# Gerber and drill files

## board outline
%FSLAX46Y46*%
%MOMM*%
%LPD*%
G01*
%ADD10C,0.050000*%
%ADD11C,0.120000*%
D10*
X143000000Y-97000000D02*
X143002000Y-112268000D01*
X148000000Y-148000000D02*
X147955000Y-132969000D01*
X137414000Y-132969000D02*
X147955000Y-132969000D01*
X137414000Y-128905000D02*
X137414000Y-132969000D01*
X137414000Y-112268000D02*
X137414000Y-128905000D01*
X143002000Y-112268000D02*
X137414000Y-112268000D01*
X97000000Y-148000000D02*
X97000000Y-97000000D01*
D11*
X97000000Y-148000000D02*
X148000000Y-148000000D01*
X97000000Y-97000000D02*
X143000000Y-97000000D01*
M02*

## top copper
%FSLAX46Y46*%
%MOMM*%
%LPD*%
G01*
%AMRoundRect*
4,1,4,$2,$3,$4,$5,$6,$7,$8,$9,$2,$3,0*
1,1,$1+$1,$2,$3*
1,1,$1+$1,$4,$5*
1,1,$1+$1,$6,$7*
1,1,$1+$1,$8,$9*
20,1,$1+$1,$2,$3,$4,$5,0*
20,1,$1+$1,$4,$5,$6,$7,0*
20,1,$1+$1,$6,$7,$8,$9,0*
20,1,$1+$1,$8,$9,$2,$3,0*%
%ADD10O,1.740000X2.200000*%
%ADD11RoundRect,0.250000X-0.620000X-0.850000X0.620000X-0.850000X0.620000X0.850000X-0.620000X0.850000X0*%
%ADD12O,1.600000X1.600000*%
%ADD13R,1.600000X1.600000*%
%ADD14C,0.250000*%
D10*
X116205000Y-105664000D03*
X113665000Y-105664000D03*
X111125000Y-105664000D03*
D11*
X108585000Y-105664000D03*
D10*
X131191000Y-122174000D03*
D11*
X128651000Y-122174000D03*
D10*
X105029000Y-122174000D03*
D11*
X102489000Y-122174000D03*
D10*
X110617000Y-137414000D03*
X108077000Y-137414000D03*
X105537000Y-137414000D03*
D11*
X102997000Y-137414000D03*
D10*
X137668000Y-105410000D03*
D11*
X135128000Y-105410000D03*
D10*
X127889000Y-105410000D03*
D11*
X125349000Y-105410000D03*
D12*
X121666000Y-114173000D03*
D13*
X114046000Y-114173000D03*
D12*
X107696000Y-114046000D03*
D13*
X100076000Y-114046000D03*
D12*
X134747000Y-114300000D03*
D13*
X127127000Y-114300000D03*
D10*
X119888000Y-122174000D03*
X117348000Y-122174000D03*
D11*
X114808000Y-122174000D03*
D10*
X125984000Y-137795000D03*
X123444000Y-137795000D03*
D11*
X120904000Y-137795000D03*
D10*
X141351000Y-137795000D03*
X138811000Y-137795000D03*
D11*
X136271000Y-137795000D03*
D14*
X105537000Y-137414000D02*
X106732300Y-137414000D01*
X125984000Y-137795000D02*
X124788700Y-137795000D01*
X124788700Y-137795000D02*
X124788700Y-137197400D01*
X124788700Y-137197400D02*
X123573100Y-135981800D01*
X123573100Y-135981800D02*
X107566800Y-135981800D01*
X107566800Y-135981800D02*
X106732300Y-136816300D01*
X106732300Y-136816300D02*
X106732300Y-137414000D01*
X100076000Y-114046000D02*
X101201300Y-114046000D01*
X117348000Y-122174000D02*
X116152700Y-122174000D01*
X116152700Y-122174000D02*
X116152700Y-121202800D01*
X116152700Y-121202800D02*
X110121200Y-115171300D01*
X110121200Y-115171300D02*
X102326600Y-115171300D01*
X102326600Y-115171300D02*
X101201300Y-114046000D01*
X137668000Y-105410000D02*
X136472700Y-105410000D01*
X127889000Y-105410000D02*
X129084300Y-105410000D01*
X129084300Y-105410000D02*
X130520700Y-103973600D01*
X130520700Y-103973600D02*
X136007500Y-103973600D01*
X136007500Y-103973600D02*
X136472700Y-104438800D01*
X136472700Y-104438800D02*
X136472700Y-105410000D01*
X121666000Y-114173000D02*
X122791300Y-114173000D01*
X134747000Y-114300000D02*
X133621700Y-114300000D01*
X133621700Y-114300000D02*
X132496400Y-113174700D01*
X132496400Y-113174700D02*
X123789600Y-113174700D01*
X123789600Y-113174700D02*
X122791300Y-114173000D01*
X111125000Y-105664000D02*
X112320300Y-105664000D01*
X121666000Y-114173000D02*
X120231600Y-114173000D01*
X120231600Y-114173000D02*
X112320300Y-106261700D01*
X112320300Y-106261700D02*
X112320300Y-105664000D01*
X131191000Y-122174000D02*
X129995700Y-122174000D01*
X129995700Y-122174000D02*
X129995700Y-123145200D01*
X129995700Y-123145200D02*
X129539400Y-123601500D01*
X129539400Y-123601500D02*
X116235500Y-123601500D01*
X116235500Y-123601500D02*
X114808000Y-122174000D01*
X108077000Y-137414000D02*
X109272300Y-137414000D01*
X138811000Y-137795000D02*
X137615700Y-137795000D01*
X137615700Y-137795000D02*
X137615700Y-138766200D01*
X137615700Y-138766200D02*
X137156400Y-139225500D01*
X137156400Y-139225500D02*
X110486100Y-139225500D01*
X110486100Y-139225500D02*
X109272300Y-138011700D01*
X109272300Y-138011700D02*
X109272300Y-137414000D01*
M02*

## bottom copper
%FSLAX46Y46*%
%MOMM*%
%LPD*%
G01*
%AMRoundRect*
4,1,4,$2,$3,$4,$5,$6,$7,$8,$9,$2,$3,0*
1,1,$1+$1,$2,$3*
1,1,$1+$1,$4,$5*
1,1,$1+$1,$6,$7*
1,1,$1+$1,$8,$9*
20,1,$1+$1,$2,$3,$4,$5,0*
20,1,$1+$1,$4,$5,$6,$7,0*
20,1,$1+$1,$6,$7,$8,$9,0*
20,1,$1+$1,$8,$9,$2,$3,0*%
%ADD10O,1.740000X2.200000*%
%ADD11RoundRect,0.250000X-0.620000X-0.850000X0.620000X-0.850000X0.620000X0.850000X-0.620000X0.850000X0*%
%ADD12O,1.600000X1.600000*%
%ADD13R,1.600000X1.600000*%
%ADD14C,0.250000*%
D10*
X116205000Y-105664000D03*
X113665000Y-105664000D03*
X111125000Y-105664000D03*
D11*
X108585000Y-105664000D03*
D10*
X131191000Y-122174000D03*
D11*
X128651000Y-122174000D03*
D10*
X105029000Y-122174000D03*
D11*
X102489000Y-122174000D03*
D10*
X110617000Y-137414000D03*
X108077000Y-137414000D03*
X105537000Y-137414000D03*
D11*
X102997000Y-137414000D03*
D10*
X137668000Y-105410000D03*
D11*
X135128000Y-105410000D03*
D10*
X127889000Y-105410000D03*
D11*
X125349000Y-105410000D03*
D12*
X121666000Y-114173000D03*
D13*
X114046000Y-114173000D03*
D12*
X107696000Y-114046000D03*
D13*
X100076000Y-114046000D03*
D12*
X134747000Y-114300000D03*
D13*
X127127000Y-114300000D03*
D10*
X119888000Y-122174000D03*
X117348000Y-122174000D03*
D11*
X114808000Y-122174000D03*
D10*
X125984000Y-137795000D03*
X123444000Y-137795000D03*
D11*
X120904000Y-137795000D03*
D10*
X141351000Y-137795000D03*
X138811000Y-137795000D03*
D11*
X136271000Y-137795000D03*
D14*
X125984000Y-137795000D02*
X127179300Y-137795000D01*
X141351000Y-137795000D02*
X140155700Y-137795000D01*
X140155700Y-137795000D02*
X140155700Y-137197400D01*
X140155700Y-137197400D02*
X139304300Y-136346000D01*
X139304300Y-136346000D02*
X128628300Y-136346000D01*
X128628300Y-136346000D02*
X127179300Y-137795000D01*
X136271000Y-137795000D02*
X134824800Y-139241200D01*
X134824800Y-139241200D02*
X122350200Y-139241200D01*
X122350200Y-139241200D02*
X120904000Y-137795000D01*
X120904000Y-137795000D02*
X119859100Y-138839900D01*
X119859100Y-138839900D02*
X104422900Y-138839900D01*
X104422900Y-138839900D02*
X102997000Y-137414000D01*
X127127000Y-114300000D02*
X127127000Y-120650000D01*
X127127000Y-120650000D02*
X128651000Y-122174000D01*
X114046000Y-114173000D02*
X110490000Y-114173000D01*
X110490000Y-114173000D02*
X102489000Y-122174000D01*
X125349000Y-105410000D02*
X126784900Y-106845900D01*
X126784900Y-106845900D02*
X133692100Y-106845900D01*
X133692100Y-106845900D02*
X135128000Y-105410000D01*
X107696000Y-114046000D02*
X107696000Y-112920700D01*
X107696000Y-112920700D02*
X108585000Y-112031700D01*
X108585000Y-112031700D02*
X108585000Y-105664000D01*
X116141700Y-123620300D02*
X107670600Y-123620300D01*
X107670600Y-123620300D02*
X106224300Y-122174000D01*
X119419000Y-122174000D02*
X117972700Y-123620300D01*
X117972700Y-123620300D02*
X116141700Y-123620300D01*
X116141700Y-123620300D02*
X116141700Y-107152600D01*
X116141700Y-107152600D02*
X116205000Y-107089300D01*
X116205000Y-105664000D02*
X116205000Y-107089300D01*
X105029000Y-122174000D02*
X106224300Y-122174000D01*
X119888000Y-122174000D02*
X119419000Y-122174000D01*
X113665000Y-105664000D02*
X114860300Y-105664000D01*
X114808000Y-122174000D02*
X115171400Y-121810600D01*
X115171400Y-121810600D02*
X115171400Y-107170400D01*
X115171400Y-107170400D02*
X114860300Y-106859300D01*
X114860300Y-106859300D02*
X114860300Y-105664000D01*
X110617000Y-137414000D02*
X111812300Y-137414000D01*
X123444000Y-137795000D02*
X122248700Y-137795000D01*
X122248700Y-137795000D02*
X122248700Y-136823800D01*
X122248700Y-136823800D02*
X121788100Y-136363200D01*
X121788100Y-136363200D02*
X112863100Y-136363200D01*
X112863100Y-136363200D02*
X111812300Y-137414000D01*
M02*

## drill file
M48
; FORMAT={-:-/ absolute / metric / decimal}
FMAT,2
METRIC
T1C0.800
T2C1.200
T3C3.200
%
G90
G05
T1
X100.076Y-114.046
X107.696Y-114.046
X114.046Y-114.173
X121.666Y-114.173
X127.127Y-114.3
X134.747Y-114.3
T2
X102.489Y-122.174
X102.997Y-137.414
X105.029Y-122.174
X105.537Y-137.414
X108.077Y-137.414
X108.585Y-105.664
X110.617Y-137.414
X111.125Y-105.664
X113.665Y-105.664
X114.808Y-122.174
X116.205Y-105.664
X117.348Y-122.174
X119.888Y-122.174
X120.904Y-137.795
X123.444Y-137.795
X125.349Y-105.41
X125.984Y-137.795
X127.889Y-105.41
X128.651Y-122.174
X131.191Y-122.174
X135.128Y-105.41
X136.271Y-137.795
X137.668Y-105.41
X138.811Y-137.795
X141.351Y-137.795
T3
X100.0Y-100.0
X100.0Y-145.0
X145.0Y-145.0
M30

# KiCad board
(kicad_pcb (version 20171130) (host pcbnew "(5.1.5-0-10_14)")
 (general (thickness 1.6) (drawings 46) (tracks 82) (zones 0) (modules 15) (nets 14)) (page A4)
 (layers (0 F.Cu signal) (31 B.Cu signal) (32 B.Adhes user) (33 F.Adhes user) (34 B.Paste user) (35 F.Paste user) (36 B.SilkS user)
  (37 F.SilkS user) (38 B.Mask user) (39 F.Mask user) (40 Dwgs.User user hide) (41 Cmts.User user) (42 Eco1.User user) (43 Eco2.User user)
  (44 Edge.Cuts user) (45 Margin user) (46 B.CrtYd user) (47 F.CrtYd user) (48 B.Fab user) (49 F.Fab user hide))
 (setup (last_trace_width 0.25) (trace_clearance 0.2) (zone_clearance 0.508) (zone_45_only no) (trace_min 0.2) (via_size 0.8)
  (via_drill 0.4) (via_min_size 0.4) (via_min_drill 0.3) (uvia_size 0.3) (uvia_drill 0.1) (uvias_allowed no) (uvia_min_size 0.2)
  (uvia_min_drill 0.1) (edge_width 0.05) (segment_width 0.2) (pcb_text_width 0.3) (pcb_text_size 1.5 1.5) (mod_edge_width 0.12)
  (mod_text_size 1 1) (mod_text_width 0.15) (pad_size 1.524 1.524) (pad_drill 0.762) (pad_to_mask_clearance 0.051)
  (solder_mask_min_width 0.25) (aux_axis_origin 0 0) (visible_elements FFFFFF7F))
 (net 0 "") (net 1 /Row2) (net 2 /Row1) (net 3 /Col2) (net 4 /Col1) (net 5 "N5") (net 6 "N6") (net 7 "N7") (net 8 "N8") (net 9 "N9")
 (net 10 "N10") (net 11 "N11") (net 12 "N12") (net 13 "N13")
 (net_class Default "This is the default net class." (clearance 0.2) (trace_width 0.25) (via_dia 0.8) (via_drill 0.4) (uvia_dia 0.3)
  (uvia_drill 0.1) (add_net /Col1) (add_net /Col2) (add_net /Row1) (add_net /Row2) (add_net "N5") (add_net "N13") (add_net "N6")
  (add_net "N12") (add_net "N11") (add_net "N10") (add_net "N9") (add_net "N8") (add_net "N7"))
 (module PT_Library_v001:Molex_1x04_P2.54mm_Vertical (layer F.Cu) (at 108.585 105.664)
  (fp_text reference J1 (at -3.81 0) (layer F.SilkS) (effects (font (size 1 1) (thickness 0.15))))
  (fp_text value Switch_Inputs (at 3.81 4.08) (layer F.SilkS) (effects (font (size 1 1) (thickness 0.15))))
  (pad 4 thru_hole oval (at 7.62 0) (size 1.74 2.2) (drill 1.2) (layers *.Cu *.Mask) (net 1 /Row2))
  (pad 3 thru_hole oval (at 5.08 0) (size 1.74 2.2) (drill 1.2) (layers *.Cu *.Mask) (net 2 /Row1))
  (pad 2 thru_hole oval (at 2.54 0) (size 1.74 2.2) (drill 1.2) (layers *.Cu *.Mask) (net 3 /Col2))
  (pad 1 thru_hole roundrect (at 0 0) (size 1.74 2.2) (drill 1.2) (layers *.Cu *.Mask) (roundrect_rratio 0.143678) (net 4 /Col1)))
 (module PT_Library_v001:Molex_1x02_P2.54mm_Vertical (layer F.Cu) (at 128.651 122.174)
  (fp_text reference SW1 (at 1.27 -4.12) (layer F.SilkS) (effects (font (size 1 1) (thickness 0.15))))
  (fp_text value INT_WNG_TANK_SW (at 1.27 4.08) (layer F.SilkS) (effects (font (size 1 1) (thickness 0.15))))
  (pad 2 thru_hole oval (at 2.54 0) (size 1.74 2.2) (drill 1.2) (layers *.Cu *.Mask) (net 2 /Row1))
  (pad 1 thru_hole roundrect (at 0 0) (size 1.74 2.2) (drill 1.2) (layers *.Cu *.Mask) (roundrect_rratio 0.143678) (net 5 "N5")))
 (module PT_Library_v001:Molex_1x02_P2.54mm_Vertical (layer F.Cu) (at 102.489 122.174)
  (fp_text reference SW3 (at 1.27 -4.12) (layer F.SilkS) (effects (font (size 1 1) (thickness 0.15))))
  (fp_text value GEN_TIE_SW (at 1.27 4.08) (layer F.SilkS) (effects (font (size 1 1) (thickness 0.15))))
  (pad 2 thru_hole oval (at 2.54 0) (size 1.74 2.2) (drill 1.2) (layers *.Cu *.Mask) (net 1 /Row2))
  (pad 1 thru_hole roundrect (at 0 0) (size 1.74 2.2) (drill 1.2) (layers *.Cu *.Mask) (roundrect_rratio 0.143678) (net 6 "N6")))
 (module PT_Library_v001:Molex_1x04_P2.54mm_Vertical (layer F.Cu) (at 102.997 137.414)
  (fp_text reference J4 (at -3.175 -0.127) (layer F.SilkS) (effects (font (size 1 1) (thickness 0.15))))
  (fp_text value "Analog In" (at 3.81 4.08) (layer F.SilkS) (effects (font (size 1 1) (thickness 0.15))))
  (pad 4 thru_hole oval (at 7.62 0) (size 1.74 2.2) (drill 1.2) (layers *.Cu *.Mask) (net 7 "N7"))
  (pad 3 thru_hole oval (at 5.08 0) (size 1.74 2.2) (drill 1.2) (layers *.Cu *.Mask) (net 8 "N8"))
  (pad 2 thru_hole oval (at 2.54 0) (size 1.74 2.2) (drill 1.2) (layers *.Cu *.Mask) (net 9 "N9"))
  (pad 1 thru_hole roundrect (at 0 0) (size 1.74 2.2) (drill 1.2) (layers *.Cu *.Mask) (roundrect_rratio 0.143678) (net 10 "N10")))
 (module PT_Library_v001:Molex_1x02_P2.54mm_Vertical (layer F.Cu) (at 135.128 105.41)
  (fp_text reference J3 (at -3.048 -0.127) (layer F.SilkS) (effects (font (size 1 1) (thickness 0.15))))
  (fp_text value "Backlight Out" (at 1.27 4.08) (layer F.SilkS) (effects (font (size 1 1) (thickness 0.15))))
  (pad 2 thru_hole oval (at 2.54 0) (size 1.74 2.2) (drill 1.2) (layers *.Cu *.Mask) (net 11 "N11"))
  (pad 1 thru_hole roundrect (at 0 0) (size 1.74 2.2) (drill 1.2) (layers *.Cu *.Mask) (roundrect_rratio 0.143678) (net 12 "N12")))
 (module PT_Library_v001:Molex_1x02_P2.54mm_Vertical (layer F.Cu) (at 125.349 105.41)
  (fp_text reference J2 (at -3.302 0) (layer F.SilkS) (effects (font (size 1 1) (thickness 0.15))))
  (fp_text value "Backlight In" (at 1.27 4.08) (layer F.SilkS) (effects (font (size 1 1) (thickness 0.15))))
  (pad 2 thru_hole oval (at 2.54 0) (size 1.74 2.2) (drill 1.2) (layers *.Cu *.Mask) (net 11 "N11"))
  (pad 1 thru_hole roundrect (at 0 0) (size 1.74 2.2) (drill 1.2) (layers *.Cu *.Mask) (roundrect_rratio 0.143678) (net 12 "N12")))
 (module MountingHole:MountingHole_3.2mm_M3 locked (layer F.Cu) (at 145 145)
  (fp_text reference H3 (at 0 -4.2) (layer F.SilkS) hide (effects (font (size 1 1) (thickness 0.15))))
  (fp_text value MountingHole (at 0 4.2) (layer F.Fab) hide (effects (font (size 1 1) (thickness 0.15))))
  (pad 1 np_thru_hole circle (at 0 0) (size 3.2 3.2) (drill 3.2) (layers *.Cu *.Mask)))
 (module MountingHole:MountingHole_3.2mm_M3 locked (layer F.Cu) (at 100 100)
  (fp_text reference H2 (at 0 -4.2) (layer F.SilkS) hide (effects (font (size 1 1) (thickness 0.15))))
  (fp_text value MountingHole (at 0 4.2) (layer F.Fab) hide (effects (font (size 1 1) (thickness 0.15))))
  (pad 1 np_thru_hole circle (at 0 0) (size 3.2 3.2) (drill 3.2) (layers *.Cu *.Mask)))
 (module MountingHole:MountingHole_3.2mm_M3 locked (layer F.Cu) (at 100 145)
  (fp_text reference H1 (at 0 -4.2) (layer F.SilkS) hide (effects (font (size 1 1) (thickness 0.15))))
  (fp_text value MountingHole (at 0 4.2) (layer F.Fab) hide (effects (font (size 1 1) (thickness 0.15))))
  (pad 1 np_thru_hole circle (at 0 0) (size 3.2 3.2) (drill 3.2) (layers *.Cu *.Mask)))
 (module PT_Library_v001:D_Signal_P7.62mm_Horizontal (layer F.Cu) (at 114.046 114.173)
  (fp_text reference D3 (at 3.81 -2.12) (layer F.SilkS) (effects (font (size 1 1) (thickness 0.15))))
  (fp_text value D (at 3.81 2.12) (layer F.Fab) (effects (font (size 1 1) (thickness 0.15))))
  (pad 2 thru_hole oval (at 7.62 0) (size 1.6 1.6) (drill 0.8) (layers *.Cu *.Mask) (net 3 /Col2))
  (pad 1 thru_hole rect (at 0 0) (size 1.6 1.6) (drill 0.8) (layers *.Cu *.Mask) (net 6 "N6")))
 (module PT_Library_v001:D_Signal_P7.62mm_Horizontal (layer F.Cu) (at 100.076 114.046)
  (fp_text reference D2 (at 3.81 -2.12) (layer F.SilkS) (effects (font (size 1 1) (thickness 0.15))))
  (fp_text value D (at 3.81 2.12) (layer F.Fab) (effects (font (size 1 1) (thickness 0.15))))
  (pad 2 thru_hole oval (at 7.62 0) (size 1.6 1.6) (drill 0.8) (layers *.Cu *.Mask) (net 4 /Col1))
  (pad 1 thru_hole rect (at 0 0) (size 1.6 1.6) (drill 0.8) (layers *.Cu *.Mask) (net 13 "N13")))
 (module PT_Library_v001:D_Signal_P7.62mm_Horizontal (layer F.Cu) (at 127.127 114.3)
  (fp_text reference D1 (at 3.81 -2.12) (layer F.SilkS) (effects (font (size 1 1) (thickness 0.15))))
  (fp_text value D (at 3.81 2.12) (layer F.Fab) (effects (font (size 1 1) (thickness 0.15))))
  (pad 2 thru_hole oval (at 7.62 0) (size 1.6 1.6) (drill 0.8) (layers *.Cu *.Mask) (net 3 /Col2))
  (pad 1 thru_hole rect (at 0 0) (size 1.6 1.6) (drill 0.8) (layers *.Cu *.Mask) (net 5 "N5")))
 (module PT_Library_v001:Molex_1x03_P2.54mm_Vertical (layer F.Cu) (at 114.808 122.174)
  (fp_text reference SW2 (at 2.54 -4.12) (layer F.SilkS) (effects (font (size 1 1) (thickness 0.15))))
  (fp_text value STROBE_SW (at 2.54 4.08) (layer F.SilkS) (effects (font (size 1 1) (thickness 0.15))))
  (pad 3 thru_hole oval (at 5.08 0) (size 1.74 2.2) (drill 1.2) (layers *.Cu *.Mask) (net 1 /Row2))
  (pad 2 thru_hole oval (at 2.54 0) (size 1.74 2.2) (drill 1.2) (layers *.Cu *.Mask) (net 13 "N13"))
  (pad 1 thru_hole roundrect (at 0 0) (size 1.74 2.2) (drill 1.2) (layers *.Cu *.Mask) (roundrect_rratio 0.143678) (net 2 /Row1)))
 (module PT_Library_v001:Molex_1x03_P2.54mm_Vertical (layer F.Cu) (at 120.904 137.795)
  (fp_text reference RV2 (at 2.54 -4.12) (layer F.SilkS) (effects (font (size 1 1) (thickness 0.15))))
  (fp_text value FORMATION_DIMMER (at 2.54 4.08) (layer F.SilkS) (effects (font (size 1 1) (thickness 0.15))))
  (pad 3 thru_hole oval (at 5.08 0) (size 1.74 2.2) (drill 1.2) (layers *.Cu *.Mask) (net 9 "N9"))
  (pad 2 thru_hole oval (at 2.54 0) (size 1.74 2.2) (drill 1.2) (layers *.Cu *.Mask) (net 7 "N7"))
  (pad 1 thru_hole roundrect (at 0 0) (size 1.74 2.2) (drill 1.2) (layers *.Cu *.Mask) (roundrect_rratio 0.143678) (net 10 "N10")))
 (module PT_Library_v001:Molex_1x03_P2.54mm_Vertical (layer F.Cu) (at 136.271 137.795)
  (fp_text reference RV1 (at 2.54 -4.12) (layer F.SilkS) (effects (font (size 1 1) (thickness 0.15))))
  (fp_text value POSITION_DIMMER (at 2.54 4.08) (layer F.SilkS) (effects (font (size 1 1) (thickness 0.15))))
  (pad 3 thru_hole oval (at 5.08 0) (size 1.74 2.2) (drill 1.2) (layers *.Cu *.Mask) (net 9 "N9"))
  (pad 2 thru_hole oval (at 2.54 0) (size 1.74 2.2) (drill 1.2) (layers *.Cu *.Mask) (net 8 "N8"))
  (pad 1 thru_hole roundrect (at 0 0) (size 1.74 2.2) (drill 1.2) (layers *.Cu *.Mask) (roundrect_rratio 0.143678) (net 10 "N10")))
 (gr_line (start 143 97) (end 143.002 112.268) (layer Edge.Cuts) (width 0.05))
 (gr_line (start 148 148) (end 147.955 132.969) (layer Edge.Cuts) (width 0.05))
 (gr_line (start 137.414 132.969) (end 147.955 132.969) (layer Edge.Cuts) (width 0.05))
 (gr_line (start 137.414 128.905) (end 137.414 132.969) (layer Edge.Cuts) (width 0.05))
 (gr_line (start 137.414 112.268) (end 137.414 128.905) (layer Edge.Cuts) (width 0.05))
 (gr_line (start 143.002 112.268) (end 137.414 112.268) (layer Edge.Cuts) (width 0.05))
 (gr_line (start 97 148) (end 97 97) (layer Edge.Cuts) (width 0.05))
 (gr_line (start 97 148) (end 148 148) (layer Edge.Cuts) (width 0.12))
 (gr_line (start 97 97) (end 143 97) (layer Edge.Cuts) (width 0.12))
 (segment (start 105.537 137.414) (end 106.7323 137.414) (width 0.25) (layer F.Cu) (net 9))
 (segment (start 125.984 137.795) (end 124.7887 137.795) (width 0.25) (layer F.Cu) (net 9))
 (segment (start 124.7887 137.795) (end 124.7887 137.1974) (width 0.25) (layer F.Cu) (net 9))
 (segment (start 124.7887 137.1974) (end 123.5731 135.9818) (width 0.25) (layer F.Cu) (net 9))
 (segment (start 123.5731 135.9818) (end 107.5668 135.9818) (width 0.25) (layer F.Cu) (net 9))
 (segment (start 107.5668 135.9818) (end 106.7323 136.8163) (width 0.25) (layer F.Cu) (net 9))
 (segment (start 106.7323 136.8163) (end 106.7323 137.414) (width 0.25) (layer F.Cu) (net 9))
 (segment (start 125.984 137.795) (end 127.1793 137.795) (width 0.25) (layer B.Cu) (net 9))
 (segment (start 141.351 137.795) (end 140.1557 137.795) (width 0.25) (layer B.Cu) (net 9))
 (segment (start 140.1557 137.795) (end 140.1557 137.1974) (width 0.25) (layer B.Cu) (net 9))
 (segment (start 140.1557 137.1974) (end 139.3043 136.346) (width 0.25) (layer B.Cu) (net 9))
 (segment (start 139.3043 136.346) (end 128.6283 136.346) (width 0.25) (layer B.Cu) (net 9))
 (segment (start 128.6283 136.346) (end 127.1793 137.795) (width 0.25) (layer B.Cu) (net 9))
 (segment (start 100.076 114.046) (end 101.2013 114.046) (width 0.25) (layer F.Cu) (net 13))
 (segment (start 117.348 122.174) (end 116.1527 122.174) (width 0.25) (layer F.Cu) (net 13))
 (segment (start 116.1527 122.174) (end 116.1527 121.2028) (width 0.25) (layer F.Cu) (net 13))
 (segment (start 116.1527 121.2028) (end 110.1212 115.1713) (width 0.25) (layer F.Cu) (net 13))
 (segment (start 110.1212 115.1713) (end 102.3266 115.1713) (width 0.25) (layer F.Cu) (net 13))
 (segment (start 102.3266 115.1713) (end 101.2013 114.046) (width 0.25) (layer F.Cu) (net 13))
 (segment (start 136.271 137.795) (end 134.8248 139.2412) (width 0.25) (layer B.Cu) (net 10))
 (segment (start 134.8248 139.2412) (end 122.3502 139.2412) (width 0.25) (layer B.Cu) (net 10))
 (segment (start 122.3502 139.2412) (end 120.904 137.795) (width 0.25) (layer B.Cu) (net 10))
 (segment (start 120.904 137.795) (end 119.8591 138.8399) (width 0.25) (layer B.Cu) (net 10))
 (segment (start 119.8591 138.8399) (end 104.4229 138.8399) (width 0.25) (layer B.Cu) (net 10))
 (segment (start 104.4229 138.8399) (end 102.997 137.414) (width 0.25) (layer B.Cu) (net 10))
 (segment (start 127.127 114.3) (end 127.127 120.65) (width 0.25) (layer B.Cu) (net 5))
 (segment (start 127.127 120.65) (end 128.651 122.174) (width 0.25) (layer B.Cu) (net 5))
 (segment (start 114.046 114.173) (end 110.49 114.173) (width 0.25) (layer B.Cu) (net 6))
 (segment (start 110.49 114.173) (end 102.489 122.174) (width 0.25) (layer B.Cu) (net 6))
 (segment (start 137.668 105.41) (end 136.4727 105.41) (width 0.25) (layer F.Cu) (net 11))
 (segment (start 127.889 105.41) (end 129.0843 105.41) (width 0.25) (layer F.Cu) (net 11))
 (segment (start 129.0843 105.41) (end 130.5207 103.9736) (width 0.25) (layer F.Cu) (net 11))
 (segment (start 130.5207 103.9736) (end 136.0075 103.9736) (width 0.25) (layer F.Cu) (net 11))
 (segment (start 136.0075 103.9736) (end 136.4727 104.4388) (width 0.25) (layer F.Cu) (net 11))
 (segment (start 136.4727 104.4388) (end 136.4727 105.41) (width 0.25) (layer F.Cu) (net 11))
 (segment (start 125.349 105.41) (end 126.7849 106.8459) (width 0.25) (layer B.Cu) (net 12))
 (segment (start 126.7849 106.8459) (end 133.6921 106.8459) (width 0.25) (layer B.Cu) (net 12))
 (segment (start 133.6921 106.8459) (end 135.128 105.41) (width 0.25) (layer B.Cu) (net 12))
 (segment (start 121.666 114.173) (end 122.7913 114.173) (width 0.25) (layer F.Cu) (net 3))
 (segment (start 134.747 114.3) (end 133.6217 114.3) (width 0.25) (layer F.Cu) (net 3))
 (segment (start 133.6217 114.3) (end 132.4964 113.1747) (width 0.25) (layer F.Cu) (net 3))
 (segment (start 132.4964 113.1747) (end 123.7896 113.1747) (width 0.25) (layer F.Cu) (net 3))
 (segment (start 123.7896 113.1747) (end 122.7913 114.173) (width 0.25) (layer F.Cu) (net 3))
 (segment (start 111.125 105.664) (end 112.3203 105.664) (width 0.25) (layer F.Cu) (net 3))
 (segment (start 121.666 114.173) (end 120.2316 114.173) (width 0.25) (layer F.Cu) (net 3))
 (segment (start 120.2316 114.173) (end 112.3203 106.2617) (width 0.25) (layer F.Cu) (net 3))
 (segment (start 112.3203 106.2617) (end 112.3203 105.664) (width 0.25) (layer F.Cu) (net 3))
 (segment (start 107.696 114.046) (end 107.696 112.9207) (width 0.25) (layer B.Cu) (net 4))
 (segment (start 107.696 112.9207) (end 108.585 112.0317) (width 0.25) (layer B.Cu) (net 4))
 (segment (start 108.585 112.0317) (end 108.585 105.664) (width 0.25) (layer B.Cu) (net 4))
 (segment (start 116.1417 123.6203) (end 107.6706 123.6203) (width 0.25) (layer B.Cu) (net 1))
 (segment (start 107.6706 123.6203) (end 106.2243 122.174) (width 0.25) (layer B.Cu) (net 1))
 (segment (start 119.419 122.174) (end 117.9727 123.6203) (width 0.25) (layer B.Cu) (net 1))
 (segment (start 117.9727 123.6203) (end 116.1417 123.6203) (width 0.25) (layer B.Cu) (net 1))
 (segment (start 116.1417 123.6203) (end 116.1417 107.1526) (width 0.25) (layer B.Cu) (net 1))
 (segment (start 116.1417 107.1526) (end 116.205 107.0893) (width 0.25) (layer B.Cu) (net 1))
 (segment (start 116.205 105.664) (end 116.205 107.0893) (width 0.25) (layer B.Cu) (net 1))
 (segment (start 105.029 122.174) (end 106.2243 122.174) (width 0.25) (layer B.Cu) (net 1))
 (segment (start 119.888 122.174) (end 119.419 122.174) (width 0.25) (layer B.Cu) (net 1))
 (segment (start 131.191 122.174) (end 129.9957 122.174) (width 0.25) (layer F.Cu) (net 2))
 (segment (start 129.9957 122.174) (end 129.9957 123.1452) (width 0.25) (layer F.Cu) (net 2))
 (segment (start 129.9957 123.1452) (end 129.5394 123.6015) (width 0.25) (layer F.Cu) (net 2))
 (segment (start 129.5394 123.6015) (end 116.2355 123.6015) (width 0.25) (layer F.Cu) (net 2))
 (segment (start 116.2355 123.6015) (end 114.808 122.174) (width 0.25) (layer F.Cu) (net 2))
 (segment (start 113.665 105.664) (end 114.8603 105.664) (width 0.25) (layer B.Cu) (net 2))
 (segment (start 114.808 122.174) (end 115.1714 121.8106) (width 0.25) (layer B.Cu) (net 2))
 (segment (start 115.1714 121.8106) (end 115.1714 107.1704) (width 0.25) (layer B.Cu) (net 2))
 (segment (start 115.1714 107.1704) (end 114.8603 106.8593) (width 0.25) (layer B.Cu) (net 2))
 (segment (start 114.8603 106.8593) (end 114.8603 105.664) (width 0.25) (layer B.Cu) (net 2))
 (segment (start 110.617 137.414) (end 111.8123 137.414) (width 0.25) (layer B.Cu) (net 7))
 (segment (start 123.444 137.795) (end 122.2487 137.795) (width 0.25) (layer B.Cu) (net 7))
 (segment (start 122.2487 137.795) (end 122.2487 136.8238) (width 0.25) (layer B.Cu) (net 7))
 (segment (start 122.2487 136.8238) (end 121.7881 136.3632) (width 0.25) (layer B.Cu) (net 7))
 (segment (start 121.7881 136.3632) (end 112.8631 136.3632) (width 0.25) (layer B.Cu) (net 7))
 (segment (start 112.8631 136.3632) (end 111.8123 137.414) (width 0.25) (layer B.Cu) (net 7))
 (segment (start 108.077 137.414) (end 109.2723 137.414) (width 0.25) (layer F.Cu) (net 8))
 (segment (start 138.811 137.795) (end 137.6157 137.795) (width 0.25) (layer F.Cu) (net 8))
 (segment (start 137.6157 137.795) (end 137.6157 138.7662) (width 0.25) (layer F.Cu) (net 8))
 (segment (start 137.6157 138.7662) (end 137.1564 139.2255) (width 0.25) (layer F.Cu) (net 8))
 (segment (start 137.1564 139.2255) (end 110.4861 139.2255) (width 0.25) (layer F.Cu) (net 8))
 (segment (start 110.4861 139.2255) (end 109.2723 138.0117) (width 0.25) (layer F.Cu) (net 8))
 (segment (start 109.2723 138.0117) (end 109.2723 137.414) (width 0.25) (layer F.Cu) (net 8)))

